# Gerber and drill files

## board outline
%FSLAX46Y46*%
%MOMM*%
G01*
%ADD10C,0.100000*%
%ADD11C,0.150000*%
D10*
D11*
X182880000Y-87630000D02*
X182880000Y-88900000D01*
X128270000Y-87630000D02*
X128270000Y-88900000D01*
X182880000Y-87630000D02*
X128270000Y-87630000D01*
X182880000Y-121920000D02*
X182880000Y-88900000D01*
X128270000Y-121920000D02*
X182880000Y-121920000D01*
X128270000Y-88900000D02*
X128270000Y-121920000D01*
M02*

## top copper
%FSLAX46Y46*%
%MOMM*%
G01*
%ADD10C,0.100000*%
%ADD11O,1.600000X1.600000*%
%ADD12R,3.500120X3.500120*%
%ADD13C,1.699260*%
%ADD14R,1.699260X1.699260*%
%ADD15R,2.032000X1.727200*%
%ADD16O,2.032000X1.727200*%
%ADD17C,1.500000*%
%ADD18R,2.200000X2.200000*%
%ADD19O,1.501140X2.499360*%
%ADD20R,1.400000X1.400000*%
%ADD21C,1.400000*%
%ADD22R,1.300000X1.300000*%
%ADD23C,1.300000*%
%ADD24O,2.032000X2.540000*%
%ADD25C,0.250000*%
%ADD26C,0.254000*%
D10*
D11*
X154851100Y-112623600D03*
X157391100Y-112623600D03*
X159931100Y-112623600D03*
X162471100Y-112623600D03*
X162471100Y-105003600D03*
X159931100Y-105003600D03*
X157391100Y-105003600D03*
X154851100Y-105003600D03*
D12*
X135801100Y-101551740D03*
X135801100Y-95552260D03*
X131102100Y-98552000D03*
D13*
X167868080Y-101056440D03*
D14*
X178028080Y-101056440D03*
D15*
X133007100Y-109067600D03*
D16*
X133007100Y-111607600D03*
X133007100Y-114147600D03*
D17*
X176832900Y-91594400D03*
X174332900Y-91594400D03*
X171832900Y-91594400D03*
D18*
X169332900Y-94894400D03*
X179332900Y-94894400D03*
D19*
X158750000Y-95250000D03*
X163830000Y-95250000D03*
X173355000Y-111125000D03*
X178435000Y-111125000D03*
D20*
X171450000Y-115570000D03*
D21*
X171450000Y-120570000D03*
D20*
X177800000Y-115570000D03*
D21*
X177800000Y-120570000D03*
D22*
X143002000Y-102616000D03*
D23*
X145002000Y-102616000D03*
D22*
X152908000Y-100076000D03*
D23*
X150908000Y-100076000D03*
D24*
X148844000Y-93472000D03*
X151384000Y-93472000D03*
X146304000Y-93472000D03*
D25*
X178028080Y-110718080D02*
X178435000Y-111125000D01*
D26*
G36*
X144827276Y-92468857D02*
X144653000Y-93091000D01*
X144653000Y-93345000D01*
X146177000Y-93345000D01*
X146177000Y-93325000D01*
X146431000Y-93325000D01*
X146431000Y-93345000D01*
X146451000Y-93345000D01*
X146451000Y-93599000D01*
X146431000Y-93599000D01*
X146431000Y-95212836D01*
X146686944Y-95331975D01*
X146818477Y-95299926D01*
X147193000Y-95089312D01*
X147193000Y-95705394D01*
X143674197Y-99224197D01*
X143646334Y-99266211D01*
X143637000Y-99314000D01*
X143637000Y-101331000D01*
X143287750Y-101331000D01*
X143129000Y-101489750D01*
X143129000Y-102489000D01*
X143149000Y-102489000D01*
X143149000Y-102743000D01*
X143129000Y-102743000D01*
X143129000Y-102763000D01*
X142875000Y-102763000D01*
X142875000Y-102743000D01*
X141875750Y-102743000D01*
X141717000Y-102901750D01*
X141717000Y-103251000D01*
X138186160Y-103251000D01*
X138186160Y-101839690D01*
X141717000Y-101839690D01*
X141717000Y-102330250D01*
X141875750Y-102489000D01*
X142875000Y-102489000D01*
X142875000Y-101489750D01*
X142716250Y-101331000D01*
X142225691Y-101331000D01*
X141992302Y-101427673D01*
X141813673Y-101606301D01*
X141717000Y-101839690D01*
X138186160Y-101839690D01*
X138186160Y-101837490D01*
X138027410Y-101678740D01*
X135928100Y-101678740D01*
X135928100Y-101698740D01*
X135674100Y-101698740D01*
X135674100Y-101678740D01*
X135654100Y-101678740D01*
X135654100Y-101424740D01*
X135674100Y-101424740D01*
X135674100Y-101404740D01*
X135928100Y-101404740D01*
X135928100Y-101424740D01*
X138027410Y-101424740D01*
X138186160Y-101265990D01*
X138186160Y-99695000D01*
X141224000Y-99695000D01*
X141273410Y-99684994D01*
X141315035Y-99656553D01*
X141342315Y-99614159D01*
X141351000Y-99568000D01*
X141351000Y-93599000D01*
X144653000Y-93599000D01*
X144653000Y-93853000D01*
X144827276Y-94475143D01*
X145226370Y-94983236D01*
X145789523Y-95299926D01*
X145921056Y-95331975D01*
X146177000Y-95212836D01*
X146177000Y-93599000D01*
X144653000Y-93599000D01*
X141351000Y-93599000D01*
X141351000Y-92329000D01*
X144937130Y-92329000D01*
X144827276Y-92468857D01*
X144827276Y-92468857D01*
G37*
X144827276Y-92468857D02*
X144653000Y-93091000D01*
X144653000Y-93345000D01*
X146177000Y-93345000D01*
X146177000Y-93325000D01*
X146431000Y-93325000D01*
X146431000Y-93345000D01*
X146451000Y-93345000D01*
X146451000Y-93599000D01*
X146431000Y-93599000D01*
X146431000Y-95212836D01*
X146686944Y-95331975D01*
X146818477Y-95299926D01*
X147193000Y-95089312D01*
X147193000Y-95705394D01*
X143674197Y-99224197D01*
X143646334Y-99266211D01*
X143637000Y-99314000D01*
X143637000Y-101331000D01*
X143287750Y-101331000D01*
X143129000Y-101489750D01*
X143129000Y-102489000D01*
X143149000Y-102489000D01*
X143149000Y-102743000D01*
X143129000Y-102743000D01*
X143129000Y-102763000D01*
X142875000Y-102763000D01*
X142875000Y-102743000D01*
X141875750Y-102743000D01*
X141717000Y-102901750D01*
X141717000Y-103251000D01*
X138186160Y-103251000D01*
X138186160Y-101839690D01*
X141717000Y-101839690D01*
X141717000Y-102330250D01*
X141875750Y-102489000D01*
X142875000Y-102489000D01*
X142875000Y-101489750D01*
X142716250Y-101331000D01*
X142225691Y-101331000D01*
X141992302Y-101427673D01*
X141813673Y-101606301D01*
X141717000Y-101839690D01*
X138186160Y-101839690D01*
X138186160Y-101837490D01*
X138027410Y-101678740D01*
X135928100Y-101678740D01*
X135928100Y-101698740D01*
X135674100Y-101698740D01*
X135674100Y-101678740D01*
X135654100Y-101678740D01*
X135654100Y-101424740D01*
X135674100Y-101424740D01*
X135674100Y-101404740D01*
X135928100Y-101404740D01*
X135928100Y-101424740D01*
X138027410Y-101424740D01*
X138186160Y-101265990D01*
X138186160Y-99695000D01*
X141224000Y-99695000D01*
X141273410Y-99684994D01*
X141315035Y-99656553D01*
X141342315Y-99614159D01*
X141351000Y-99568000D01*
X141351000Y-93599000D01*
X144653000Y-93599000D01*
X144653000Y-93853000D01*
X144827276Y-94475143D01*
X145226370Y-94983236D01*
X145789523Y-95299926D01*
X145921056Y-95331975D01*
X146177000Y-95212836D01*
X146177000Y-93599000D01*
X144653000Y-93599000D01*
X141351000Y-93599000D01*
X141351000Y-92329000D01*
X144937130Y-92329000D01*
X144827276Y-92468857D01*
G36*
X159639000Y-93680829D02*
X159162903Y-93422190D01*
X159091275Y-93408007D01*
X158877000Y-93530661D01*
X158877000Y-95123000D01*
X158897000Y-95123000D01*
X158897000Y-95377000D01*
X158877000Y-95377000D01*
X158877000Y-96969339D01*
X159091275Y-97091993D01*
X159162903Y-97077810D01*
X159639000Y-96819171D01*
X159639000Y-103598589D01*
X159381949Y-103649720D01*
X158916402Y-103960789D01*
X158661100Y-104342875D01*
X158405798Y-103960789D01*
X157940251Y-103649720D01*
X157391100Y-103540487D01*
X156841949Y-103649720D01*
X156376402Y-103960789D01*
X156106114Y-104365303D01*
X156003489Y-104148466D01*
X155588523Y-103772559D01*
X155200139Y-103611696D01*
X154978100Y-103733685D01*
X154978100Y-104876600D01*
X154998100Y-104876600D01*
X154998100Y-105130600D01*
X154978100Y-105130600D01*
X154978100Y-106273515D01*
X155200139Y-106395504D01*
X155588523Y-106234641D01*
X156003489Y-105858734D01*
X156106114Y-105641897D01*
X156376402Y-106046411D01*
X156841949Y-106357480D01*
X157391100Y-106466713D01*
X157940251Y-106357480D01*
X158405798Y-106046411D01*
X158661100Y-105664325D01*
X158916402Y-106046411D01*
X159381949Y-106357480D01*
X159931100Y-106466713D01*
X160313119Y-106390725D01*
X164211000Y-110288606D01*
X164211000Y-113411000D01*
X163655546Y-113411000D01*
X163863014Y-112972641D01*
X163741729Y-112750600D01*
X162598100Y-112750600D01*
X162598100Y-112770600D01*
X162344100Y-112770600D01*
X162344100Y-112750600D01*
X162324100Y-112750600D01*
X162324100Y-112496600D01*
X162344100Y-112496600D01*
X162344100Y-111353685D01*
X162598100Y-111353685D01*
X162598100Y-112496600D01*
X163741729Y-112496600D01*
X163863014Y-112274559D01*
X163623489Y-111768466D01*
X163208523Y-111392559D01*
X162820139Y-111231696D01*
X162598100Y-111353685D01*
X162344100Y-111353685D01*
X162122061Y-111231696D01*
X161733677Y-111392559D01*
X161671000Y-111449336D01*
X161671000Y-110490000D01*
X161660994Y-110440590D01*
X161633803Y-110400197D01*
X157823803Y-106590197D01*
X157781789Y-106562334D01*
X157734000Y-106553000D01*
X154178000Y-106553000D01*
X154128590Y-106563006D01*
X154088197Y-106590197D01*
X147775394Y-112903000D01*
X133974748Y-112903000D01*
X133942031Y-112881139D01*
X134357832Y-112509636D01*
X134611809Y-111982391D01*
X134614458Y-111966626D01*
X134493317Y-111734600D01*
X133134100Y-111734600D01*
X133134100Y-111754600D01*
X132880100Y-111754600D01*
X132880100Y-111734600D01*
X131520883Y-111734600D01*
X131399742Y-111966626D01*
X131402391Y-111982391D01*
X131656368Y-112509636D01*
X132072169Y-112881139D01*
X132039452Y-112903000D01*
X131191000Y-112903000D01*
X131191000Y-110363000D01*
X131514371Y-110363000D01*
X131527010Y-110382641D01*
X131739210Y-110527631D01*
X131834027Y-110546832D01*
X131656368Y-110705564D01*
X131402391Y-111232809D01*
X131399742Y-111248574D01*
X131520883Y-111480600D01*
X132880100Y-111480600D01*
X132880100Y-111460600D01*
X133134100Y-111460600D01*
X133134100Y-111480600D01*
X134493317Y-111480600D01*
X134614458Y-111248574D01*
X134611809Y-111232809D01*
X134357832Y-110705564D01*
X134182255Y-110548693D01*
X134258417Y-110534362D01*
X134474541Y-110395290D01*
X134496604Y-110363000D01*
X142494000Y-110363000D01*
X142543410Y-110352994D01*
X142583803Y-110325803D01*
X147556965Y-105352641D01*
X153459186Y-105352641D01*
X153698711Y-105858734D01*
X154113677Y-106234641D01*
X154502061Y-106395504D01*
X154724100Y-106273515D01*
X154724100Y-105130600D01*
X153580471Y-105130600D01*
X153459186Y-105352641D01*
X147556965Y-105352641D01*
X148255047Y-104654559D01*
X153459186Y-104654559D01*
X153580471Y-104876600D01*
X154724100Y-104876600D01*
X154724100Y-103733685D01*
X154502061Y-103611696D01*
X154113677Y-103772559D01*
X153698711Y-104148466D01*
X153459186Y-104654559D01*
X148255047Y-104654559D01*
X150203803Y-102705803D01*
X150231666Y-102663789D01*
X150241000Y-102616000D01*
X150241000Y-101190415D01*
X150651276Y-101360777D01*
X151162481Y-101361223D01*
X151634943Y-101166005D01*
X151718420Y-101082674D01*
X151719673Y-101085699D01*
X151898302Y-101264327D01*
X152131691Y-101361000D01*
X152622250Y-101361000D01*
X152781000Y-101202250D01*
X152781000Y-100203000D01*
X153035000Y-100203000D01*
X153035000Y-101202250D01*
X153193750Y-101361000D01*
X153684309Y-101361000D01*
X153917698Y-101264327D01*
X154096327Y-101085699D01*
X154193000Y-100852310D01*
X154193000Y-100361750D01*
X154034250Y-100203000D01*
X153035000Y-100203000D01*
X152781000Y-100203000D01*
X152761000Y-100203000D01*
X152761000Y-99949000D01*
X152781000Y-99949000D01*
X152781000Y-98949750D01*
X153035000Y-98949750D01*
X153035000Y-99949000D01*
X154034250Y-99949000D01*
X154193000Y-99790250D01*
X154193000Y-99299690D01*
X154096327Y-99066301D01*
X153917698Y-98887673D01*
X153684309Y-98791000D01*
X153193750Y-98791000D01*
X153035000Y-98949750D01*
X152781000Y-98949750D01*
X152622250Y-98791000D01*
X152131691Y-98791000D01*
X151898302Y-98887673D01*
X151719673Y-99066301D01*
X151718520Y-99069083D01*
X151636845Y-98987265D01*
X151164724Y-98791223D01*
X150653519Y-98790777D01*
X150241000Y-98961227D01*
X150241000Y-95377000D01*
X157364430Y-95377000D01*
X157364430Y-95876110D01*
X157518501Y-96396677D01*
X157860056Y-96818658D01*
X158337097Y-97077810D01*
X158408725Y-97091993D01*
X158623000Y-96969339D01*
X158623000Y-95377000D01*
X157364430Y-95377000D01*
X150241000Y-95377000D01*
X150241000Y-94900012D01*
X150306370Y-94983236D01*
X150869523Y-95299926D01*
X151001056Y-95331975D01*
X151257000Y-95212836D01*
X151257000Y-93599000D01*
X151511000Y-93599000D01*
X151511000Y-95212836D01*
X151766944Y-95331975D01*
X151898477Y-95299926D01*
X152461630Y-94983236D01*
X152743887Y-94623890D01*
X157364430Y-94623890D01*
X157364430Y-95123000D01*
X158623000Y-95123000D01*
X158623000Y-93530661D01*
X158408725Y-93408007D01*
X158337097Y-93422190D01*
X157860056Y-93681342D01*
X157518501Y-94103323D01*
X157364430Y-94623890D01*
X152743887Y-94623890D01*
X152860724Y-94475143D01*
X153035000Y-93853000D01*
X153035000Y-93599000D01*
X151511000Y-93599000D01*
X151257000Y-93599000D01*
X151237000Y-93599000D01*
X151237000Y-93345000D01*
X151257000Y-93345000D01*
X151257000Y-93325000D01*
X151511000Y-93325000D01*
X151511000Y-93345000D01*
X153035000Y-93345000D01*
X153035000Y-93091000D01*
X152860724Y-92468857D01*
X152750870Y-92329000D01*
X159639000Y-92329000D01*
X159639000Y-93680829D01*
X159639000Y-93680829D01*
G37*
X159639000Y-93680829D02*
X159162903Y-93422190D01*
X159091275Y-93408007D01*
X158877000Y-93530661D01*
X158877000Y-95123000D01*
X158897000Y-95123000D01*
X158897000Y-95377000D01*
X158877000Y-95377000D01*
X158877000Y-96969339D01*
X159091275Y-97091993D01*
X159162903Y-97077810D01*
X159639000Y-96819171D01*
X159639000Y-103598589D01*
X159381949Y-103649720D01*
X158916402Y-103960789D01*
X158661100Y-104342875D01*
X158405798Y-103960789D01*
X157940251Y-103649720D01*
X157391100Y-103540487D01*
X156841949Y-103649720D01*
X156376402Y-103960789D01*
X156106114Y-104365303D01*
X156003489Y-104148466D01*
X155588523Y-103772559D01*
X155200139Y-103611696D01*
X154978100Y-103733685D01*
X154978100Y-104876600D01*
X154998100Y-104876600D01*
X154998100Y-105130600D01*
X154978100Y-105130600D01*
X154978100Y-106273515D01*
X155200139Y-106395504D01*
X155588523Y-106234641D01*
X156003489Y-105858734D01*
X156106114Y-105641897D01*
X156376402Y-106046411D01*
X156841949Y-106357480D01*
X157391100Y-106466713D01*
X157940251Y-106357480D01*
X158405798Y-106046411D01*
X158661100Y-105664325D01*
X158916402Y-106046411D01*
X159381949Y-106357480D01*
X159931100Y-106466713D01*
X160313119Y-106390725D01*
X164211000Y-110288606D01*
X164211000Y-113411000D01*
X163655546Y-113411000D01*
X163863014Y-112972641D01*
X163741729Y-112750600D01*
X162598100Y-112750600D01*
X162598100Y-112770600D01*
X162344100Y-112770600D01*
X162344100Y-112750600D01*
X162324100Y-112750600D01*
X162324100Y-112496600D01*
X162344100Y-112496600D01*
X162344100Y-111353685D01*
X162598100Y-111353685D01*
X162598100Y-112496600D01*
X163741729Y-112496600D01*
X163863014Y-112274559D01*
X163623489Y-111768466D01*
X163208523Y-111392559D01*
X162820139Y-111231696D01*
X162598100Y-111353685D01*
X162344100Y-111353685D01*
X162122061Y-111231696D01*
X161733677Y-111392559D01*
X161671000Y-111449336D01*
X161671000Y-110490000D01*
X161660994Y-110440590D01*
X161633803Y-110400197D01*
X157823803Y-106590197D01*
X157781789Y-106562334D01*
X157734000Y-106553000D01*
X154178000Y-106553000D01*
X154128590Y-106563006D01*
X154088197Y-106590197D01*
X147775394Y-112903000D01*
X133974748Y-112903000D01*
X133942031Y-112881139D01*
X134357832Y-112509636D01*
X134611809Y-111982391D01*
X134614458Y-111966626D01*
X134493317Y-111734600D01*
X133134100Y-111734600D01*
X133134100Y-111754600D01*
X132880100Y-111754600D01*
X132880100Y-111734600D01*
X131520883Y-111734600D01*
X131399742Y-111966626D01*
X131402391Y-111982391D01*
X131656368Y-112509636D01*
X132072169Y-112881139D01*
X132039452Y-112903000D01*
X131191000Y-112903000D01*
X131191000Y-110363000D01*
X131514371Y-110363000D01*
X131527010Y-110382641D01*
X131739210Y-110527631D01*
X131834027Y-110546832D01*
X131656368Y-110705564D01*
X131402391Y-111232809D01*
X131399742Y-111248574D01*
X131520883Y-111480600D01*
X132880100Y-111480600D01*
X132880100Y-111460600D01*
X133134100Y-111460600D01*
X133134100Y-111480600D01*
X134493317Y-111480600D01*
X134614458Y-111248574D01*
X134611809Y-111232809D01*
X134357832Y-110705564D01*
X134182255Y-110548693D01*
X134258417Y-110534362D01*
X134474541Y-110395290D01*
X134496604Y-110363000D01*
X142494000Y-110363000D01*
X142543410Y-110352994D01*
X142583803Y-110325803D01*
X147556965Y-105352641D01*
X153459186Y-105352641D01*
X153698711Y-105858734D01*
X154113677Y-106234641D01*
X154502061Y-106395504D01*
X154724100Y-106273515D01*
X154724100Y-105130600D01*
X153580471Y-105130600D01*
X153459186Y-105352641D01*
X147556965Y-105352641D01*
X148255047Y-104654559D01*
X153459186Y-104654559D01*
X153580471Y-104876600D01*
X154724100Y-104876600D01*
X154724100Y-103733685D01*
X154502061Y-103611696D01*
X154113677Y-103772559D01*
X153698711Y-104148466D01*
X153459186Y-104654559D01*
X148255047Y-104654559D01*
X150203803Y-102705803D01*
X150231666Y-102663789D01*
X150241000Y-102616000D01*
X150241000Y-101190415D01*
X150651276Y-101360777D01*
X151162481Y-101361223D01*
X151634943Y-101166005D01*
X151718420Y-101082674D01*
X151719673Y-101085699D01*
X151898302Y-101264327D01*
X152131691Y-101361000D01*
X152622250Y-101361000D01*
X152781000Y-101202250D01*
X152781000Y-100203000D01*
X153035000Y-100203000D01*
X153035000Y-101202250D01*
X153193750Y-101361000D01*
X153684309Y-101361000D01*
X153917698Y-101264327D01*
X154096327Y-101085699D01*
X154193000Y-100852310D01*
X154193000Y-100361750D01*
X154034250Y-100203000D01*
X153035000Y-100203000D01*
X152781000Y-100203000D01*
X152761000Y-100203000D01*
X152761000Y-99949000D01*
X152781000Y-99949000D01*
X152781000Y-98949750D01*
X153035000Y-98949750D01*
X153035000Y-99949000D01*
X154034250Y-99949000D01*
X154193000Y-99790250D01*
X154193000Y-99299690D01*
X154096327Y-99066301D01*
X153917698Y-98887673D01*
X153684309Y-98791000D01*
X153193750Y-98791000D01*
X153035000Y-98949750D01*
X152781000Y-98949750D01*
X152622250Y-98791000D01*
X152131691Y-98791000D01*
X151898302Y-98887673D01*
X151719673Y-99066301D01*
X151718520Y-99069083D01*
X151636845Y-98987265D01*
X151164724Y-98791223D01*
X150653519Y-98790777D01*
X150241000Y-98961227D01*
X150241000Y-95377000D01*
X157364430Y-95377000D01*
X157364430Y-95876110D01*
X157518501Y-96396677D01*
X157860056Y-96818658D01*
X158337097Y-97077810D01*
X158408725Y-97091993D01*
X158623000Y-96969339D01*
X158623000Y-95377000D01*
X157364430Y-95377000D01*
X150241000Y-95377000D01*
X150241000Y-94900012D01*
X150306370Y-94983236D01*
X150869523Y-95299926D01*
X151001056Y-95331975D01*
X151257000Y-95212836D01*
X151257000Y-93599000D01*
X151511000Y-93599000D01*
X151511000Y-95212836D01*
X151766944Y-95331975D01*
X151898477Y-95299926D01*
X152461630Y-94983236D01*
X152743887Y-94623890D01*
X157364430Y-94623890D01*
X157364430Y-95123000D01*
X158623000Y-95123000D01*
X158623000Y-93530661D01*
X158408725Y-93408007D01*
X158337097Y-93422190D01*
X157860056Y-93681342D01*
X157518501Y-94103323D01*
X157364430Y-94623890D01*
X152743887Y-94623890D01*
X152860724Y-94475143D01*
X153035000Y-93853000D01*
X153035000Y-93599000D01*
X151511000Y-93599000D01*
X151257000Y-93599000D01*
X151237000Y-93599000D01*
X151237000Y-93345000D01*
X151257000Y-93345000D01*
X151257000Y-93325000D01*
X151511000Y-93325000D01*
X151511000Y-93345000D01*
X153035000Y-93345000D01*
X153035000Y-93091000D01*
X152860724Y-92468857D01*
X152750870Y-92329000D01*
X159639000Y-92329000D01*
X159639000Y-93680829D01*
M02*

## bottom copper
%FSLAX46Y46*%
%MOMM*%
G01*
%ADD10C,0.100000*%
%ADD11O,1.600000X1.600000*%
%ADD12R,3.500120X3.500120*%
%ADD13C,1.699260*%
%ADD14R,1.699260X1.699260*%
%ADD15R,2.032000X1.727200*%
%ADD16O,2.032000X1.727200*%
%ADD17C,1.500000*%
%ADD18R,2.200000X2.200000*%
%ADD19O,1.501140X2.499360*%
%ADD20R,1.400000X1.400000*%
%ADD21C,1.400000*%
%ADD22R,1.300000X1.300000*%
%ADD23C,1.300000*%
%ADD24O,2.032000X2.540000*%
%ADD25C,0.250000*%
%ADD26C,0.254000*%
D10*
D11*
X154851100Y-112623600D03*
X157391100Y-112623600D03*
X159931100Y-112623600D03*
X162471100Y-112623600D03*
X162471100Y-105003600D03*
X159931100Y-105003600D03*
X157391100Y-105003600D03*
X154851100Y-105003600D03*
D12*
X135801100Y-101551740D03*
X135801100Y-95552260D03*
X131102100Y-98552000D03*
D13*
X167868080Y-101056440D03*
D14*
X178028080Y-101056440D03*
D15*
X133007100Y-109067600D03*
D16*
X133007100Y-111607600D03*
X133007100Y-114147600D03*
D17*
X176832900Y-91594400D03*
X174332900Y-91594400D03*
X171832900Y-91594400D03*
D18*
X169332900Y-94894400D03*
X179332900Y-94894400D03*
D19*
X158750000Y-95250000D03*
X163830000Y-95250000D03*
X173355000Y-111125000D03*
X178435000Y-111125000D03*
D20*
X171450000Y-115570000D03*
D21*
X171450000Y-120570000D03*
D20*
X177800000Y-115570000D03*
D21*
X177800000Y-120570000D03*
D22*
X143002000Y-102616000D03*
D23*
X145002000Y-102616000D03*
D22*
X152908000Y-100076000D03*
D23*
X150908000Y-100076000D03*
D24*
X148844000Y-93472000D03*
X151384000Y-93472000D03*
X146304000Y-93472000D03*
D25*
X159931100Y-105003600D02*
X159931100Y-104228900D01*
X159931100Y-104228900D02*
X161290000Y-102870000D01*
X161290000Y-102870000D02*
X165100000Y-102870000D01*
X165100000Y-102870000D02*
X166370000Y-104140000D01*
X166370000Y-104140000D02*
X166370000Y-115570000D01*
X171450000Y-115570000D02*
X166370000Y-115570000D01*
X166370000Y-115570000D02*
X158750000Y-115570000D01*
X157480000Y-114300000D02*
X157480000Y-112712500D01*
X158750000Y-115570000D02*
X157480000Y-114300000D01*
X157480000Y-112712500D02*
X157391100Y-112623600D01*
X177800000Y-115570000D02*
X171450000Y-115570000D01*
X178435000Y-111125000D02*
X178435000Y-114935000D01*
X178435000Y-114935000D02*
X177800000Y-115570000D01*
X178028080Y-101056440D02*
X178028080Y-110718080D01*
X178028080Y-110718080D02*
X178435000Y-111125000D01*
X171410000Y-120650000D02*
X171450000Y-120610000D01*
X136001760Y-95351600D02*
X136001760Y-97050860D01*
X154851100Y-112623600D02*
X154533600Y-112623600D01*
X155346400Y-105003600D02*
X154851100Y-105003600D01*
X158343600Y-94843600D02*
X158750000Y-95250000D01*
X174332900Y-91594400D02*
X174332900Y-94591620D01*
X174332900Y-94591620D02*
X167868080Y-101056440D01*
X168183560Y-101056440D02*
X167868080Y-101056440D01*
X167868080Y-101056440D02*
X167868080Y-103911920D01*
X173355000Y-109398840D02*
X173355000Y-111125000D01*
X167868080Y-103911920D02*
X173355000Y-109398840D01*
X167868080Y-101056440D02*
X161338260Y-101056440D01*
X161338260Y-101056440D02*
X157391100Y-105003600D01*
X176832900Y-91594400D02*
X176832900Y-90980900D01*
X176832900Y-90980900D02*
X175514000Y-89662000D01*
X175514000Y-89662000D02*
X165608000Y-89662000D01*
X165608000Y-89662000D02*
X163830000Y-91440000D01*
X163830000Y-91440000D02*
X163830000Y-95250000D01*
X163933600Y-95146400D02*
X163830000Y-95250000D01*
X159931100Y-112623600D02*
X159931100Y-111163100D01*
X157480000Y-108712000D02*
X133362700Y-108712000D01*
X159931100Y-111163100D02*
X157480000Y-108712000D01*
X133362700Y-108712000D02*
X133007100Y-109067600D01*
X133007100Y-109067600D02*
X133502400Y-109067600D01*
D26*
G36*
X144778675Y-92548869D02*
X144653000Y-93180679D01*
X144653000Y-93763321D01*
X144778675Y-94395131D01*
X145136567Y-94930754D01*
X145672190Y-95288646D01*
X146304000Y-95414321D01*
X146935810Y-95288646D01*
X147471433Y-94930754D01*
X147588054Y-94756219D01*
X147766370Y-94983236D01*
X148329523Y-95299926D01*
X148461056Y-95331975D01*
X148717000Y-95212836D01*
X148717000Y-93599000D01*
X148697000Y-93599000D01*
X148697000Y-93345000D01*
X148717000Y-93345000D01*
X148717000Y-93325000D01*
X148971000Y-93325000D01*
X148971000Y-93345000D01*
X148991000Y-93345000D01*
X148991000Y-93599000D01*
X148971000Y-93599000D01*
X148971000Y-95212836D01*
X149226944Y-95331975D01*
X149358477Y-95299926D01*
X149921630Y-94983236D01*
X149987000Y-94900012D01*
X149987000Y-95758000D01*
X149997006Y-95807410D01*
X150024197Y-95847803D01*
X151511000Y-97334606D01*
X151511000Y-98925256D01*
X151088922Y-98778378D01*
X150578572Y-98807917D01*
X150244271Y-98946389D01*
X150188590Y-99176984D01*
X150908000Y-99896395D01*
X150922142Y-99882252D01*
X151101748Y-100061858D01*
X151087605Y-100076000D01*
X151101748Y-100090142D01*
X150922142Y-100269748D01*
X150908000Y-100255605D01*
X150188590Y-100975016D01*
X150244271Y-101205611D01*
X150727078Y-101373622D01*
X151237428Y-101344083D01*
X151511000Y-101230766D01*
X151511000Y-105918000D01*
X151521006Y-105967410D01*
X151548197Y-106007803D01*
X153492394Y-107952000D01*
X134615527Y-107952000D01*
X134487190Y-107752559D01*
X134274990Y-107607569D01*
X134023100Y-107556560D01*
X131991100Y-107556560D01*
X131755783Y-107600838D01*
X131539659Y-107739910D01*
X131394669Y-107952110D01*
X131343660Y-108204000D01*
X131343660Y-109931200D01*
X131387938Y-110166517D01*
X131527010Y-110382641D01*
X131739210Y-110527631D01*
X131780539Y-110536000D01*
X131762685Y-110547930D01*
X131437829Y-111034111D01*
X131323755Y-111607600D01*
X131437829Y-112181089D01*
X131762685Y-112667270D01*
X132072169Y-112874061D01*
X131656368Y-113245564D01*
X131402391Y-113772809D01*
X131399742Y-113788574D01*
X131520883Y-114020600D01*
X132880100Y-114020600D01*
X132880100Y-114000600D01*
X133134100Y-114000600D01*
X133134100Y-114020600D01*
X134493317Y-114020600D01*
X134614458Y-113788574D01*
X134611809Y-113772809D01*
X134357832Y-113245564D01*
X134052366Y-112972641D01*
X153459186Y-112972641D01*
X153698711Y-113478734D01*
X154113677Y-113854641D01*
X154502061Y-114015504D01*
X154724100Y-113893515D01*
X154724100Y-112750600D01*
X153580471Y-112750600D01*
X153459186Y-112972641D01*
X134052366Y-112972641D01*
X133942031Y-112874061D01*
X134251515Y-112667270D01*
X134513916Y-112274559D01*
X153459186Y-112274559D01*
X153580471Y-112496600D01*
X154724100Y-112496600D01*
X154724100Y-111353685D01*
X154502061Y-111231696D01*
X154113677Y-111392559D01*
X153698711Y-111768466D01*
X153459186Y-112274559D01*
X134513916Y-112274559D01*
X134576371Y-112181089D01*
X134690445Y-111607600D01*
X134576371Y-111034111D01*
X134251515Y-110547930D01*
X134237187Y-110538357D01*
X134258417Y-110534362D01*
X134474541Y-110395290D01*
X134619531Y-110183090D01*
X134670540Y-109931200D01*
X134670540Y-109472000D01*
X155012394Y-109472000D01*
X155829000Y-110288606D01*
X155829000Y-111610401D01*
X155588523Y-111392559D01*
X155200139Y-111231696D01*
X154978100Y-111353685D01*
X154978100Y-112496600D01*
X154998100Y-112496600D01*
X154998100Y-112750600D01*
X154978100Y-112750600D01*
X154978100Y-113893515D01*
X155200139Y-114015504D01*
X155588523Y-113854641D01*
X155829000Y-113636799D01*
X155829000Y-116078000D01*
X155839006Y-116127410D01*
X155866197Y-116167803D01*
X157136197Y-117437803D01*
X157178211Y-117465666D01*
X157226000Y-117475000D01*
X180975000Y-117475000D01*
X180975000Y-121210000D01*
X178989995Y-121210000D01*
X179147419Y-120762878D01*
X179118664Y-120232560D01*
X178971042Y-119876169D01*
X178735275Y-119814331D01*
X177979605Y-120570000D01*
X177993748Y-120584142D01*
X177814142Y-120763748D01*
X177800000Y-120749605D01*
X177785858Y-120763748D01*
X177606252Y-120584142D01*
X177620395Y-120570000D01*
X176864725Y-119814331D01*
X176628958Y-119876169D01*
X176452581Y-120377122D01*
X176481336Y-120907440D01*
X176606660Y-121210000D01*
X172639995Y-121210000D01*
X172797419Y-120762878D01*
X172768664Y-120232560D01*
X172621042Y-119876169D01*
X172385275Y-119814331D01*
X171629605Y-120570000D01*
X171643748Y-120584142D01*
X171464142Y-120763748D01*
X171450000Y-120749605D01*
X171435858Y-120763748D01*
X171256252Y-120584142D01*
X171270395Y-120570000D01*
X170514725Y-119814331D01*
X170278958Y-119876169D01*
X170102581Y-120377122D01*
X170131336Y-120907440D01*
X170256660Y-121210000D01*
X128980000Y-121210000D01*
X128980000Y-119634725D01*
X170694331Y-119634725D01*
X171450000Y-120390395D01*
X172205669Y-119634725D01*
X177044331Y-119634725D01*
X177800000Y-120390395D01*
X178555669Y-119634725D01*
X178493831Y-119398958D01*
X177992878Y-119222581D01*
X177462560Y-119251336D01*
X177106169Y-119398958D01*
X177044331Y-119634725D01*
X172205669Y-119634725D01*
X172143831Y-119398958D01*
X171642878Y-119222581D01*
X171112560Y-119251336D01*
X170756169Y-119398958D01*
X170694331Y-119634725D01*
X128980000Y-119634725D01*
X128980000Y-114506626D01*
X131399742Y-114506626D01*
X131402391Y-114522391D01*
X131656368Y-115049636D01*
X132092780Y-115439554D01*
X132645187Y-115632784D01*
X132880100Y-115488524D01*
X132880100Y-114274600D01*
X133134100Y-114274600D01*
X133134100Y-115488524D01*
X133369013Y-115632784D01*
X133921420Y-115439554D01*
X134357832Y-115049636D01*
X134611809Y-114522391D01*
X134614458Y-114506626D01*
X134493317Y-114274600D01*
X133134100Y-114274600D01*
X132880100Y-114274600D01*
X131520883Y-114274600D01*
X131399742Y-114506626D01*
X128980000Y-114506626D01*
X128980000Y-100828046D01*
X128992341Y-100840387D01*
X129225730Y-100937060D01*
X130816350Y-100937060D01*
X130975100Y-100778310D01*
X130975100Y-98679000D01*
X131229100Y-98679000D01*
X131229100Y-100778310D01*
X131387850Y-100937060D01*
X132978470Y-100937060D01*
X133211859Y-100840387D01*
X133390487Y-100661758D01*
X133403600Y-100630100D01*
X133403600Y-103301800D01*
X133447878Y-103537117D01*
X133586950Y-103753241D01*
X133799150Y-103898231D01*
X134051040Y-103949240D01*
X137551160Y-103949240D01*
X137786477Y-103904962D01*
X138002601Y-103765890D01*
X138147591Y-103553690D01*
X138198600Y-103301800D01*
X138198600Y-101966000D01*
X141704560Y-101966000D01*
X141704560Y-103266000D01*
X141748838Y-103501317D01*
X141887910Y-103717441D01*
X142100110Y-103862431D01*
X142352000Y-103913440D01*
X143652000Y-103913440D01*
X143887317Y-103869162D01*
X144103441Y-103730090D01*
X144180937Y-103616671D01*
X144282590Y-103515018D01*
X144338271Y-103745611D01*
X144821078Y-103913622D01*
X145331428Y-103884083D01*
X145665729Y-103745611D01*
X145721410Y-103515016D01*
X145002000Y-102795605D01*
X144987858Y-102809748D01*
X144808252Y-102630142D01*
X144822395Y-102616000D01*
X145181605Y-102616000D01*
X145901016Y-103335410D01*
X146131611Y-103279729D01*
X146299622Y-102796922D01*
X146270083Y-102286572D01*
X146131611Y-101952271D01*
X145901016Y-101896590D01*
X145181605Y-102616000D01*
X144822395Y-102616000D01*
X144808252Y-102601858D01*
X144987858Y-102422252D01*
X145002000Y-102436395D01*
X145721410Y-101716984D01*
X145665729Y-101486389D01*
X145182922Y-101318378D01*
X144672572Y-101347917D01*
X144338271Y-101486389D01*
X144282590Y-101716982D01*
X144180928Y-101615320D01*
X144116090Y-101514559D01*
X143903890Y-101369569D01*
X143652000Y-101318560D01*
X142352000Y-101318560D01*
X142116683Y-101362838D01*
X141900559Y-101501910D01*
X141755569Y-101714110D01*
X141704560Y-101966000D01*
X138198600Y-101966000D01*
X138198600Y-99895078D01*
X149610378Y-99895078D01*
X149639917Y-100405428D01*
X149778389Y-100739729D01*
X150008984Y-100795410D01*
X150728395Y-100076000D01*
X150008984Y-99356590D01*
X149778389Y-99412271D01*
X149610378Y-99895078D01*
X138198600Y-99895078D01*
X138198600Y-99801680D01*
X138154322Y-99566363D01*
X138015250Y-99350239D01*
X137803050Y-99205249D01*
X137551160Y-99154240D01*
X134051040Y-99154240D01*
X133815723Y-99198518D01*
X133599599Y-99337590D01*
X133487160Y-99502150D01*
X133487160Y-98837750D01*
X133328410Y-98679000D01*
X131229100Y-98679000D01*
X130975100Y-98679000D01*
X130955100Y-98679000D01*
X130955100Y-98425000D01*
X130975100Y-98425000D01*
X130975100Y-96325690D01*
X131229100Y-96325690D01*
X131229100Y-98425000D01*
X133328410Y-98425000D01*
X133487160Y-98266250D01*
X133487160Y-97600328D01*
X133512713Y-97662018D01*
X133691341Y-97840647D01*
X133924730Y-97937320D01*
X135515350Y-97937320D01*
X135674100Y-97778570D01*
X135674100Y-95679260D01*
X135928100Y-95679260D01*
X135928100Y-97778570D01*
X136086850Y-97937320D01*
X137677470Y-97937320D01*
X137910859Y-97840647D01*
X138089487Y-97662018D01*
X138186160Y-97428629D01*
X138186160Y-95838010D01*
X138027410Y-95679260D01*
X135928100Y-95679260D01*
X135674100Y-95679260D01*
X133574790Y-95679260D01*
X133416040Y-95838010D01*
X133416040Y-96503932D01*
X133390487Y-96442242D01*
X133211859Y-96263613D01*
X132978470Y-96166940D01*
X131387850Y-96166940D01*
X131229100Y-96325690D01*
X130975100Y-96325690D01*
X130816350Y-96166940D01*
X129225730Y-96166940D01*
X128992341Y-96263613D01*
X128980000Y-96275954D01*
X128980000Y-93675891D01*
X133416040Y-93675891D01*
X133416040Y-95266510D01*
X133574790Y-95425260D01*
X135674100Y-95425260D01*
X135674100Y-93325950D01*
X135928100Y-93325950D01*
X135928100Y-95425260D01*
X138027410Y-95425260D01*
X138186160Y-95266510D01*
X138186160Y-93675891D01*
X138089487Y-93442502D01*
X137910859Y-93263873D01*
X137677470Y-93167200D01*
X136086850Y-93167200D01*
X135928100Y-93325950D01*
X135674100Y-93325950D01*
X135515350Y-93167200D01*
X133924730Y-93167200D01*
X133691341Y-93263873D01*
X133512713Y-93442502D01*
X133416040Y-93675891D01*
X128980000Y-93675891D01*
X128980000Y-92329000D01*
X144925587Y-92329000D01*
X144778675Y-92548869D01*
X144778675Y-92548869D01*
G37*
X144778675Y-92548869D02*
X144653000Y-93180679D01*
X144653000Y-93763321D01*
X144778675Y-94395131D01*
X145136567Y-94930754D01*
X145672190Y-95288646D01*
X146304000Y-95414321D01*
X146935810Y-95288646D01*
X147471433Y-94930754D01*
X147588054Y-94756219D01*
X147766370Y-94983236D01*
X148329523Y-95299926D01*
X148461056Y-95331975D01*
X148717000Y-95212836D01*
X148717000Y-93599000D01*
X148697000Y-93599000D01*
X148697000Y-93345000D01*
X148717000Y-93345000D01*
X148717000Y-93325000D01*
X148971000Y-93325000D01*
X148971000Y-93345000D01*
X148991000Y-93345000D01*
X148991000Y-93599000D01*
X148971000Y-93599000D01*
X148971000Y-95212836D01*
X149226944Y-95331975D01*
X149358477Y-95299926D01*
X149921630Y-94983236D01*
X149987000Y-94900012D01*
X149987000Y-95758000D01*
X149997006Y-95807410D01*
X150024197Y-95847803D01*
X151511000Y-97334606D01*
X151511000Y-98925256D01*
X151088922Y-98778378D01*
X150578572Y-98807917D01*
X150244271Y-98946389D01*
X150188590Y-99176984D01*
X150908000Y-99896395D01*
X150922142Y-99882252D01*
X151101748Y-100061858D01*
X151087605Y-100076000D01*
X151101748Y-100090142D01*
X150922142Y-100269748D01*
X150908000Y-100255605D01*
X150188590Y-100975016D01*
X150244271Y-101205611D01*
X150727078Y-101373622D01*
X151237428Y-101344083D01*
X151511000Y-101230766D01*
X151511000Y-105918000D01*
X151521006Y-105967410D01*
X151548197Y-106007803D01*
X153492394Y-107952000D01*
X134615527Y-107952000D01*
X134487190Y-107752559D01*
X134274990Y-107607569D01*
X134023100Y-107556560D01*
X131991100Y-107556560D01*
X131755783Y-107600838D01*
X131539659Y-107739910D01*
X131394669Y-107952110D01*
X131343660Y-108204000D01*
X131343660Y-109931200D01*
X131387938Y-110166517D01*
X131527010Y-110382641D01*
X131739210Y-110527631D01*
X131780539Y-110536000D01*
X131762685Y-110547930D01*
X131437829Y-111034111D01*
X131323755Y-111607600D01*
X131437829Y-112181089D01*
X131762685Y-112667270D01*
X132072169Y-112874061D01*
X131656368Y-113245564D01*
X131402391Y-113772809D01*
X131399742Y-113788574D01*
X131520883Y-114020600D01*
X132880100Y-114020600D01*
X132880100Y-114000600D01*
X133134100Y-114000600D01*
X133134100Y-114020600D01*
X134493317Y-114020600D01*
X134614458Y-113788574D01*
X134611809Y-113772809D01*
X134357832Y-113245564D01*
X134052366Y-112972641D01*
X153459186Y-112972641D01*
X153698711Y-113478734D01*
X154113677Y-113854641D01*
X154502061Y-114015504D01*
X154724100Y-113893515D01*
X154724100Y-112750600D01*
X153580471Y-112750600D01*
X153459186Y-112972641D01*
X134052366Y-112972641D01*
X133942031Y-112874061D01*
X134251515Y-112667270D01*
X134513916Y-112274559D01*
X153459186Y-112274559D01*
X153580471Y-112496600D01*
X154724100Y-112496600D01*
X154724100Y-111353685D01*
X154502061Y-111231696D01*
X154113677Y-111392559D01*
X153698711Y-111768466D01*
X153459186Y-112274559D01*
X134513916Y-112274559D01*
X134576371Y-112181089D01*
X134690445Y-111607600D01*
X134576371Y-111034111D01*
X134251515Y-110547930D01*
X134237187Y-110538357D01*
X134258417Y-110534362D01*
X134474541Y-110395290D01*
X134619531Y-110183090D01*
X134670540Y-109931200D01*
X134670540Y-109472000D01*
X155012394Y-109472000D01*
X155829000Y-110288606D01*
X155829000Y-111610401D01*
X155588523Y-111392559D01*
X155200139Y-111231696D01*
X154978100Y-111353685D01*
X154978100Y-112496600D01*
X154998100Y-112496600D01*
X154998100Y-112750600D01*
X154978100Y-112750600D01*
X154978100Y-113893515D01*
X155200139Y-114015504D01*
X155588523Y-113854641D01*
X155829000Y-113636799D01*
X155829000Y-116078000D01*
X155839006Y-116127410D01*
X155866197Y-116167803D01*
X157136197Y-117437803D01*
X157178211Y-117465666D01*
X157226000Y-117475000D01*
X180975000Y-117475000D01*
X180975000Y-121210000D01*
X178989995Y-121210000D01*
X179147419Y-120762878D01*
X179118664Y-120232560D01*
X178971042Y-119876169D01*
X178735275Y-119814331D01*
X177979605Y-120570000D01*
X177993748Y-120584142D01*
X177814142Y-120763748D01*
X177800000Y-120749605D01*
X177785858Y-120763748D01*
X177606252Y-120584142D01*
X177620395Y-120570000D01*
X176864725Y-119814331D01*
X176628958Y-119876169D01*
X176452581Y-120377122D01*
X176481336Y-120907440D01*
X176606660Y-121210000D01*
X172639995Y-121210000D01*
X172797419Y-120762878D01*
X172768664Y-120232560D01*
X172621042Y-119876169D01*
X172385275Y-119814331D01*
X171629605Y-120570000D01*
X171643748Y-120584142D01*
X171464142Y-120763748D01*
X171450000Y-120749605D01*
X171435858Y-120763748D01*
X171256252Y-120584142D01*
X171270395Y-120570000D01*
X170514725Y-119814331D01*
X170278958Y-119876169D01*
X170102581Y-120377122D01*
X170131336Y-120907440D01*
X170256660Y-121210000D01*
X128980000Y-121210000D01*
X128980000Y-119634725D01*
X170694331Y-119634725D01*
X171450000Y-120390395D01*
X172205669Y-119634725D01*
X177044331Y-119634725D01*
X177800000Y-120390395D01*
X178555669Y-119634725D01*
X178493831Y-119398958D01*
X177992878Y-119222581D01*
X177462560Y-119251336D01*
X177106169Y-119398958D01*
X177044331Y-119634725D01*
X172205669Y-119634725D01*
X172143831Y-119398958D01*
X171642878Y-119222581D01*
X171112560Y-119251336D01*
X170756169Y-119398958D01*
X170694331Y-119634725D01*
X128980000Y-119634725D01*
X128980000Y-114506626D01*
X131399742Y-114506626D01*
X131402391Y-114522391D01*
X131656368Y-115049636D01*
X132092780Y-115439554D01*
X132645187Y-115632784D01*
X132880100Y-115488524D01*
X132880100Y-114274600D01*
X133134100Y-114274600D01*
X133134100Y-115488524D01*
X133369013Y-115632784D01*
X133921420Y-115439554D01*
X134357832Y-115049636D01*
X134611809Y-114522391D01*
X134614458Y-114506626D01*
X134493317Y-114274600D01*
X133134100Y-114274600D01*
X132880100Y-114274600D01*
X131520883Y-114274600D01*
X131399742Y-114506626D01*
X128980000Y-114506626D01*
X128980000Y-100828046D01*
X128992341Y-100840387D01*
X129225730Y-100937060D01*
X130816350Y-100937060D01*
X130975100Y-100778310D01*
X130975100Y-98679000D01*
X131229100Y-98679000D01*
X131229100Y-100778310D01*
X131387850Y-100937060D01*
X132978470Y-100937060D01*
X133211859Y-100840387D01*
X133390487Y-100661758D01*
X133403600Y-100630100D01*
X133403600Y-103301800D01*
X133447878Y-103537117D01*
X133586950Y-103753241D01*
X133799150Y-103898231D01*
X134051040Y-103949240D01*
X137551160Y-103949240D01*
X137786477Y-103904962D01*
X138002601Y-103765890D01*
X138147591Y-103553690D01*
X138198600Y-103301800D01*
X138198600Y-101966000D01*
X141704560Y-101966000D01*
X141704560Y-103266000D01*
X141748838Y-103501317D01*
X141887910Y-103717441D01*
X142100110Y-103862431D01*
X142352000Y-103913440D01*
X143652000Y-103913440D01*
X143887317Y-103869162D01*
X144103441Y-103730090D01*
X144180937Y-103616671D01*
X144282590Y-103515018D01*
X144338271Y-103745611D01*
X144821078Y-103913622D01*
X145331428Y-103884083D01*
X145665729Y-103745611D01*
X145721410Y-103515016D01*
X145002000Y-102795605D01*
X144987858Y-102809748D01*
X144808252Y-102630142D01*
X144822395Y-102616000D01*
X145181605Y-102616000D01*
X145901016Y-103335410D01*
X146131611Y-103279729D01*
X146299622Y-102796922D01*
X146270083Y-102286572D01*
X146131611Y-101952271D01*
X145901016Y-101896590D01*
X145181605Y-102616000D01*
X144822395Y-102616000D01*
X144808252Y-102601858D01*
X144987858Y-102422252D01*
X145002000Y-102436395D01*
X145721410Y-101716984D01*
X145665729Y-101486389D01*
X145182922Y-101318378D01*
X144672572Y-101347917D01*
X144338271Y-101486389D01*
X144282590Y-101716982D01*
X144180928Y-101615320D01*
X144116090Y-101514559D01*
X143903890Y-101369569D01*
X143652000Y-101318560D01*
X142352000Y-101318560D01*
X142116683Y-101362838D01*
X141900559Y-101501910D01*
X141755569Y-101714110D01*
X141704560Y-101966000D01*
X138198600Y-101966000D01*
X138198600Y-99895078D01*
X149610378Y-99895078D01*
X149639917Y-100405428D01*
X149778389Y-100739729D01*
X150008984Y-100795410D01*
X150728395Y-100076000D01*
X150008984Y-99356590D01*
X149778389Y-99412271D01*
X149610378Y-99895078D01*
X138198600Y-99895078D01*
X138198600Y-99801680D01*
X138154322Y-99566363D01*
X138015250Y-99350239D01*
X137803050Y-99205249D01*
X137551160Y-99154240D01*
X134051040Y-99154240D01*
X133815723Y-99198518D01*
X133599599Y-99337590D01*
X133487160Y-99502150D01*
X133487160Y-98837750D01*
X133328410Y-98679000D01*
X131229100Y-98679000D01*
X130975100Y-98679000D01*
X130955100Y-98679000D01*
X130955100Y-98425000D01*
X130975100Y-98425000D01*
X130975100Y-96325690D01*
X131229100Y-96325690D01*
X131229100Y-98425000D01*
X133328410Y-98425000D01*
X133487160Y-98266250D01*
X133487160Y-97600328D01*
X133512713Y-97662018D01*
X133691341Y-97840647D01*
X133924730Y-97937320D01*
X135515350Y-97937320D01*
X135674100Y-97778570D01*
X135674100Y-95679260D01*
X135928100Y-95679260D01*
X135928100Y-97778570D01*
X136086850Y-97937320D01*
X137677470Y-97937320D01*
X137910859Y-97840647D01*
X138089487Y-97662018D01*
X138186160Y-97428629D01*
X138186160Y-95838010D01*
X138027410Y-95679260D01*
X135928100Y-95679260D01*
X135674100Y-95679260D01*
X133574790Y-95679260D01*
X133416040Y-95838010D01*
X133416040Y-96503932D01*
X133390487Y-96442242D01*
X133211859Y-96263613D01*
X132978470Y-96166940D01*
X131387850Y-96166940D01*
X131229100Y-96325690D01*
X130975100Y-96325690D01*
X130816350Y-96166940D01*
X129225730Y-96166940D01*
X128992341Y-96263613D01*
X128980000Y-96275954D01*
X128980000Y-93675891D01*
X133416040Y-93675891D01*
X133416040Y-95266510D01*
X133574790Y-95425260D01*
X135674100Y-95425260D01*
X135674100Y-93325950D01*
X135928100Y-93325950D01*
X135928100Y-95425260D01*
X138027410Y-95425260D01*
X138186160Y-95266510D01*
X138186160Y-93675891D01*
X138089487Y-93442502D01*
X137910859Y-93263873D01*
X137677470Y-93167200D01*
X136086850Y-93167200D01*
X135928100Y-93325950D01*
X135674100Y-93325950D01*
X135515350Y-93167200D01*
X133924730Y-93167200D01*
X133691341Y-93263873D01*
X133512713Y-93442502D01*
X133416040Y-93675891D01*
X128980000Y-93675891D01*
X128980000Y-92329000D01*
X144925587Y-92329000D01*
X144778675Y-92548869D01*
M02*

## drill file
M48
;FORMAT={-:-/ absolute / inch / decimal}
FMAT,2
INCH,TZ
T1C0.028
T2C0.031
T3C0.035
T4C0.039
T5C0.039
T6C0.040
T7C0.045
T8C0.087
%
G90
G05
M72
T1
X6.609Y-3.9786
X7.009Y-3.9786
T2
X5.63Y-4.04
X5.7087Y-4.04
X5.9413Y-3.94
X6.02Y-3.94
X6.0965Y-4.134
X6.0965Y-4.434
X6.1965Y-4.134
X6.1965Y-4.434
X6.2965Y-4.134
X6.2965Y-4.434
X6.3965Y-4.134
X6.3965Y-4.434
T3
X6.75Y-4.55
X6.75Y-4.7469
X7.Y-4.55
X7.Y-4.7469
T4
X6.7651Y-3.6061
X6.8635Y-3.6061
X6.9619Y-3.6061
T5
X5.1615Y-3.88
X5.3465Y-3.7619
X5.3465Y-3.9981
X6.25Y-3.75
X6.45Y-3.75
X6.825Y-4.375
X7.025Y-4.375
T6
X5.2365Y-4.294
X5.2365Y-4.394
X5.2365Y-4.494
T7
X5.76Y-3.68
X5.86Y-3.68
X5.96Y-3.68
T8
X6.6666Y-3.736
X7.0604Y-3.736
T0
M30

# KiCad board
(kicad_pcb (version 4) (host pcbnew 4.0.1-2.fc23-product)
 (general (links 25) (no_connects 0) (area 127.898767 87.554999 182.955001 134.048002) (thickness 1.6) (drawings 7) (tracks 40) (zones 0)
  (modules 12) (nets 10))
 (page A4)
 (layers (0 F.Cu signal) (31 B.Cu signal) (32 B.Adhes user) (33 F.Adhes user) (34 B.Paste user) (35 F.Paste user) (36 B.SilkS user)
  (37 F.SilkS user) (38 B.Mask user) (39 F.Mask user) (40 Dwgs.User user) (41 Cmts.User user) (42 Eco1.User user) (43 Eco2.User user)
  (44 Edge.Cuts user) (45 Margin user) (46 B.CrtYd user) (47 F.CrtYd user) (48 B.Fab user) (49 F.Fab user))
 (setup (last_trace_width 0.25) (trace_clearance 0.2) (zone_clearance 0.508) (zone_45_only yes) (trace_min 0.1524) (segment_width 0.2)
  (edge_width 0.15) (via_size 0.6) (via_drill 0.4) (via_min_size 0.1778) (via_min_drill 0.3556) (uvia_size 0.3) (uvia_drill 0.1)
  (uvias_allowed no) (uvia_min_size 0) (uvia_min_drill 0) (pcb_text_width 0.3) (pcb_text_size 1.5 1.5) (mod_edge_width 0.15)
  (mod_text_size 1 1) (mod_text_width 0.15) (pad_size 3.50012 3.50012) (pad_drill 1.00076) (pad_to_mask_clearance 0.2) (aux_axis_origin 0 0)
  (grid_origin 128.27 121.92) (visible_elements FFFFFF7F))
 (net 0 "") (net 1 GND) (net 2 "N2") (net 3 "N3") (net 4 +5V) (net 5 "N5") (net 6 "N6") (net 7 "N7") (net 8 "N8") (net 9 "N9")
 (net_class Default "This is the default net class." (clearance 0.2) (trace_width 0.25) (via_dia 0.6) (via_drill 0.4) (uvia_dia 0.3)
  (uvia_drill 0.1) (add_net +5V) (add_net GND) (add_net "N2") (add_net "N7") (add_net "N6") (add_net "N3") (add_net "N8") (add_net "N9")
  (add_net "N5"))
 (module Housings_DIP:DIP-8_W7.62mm (layer F.Cu) (at 154.8511 112.6236 90)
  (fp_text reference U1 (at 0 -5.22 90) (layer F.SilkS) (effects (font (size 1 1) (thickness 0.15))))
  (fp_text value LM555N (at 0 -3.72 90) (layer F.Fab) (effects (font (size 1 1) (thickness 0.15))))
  (pad 1 thru_hole oval (at 0 0 90) (size 1.6 1.6) (drill 0.8) (layers *.Cu *.Mask F.SilkS) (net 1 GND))
  (pad 2 thru_hole oval (at 0 2.54 90) (size 1.6 1.6) (drill 0.8) (layers *.Cu *.Mask F.SilkS) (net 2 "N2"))
  (pad 3 thru_hole oval (at 0 5.08 90) (size 1.6 1.6) (drill 0.8) (layers *.Cu *.Mask F.SilkS) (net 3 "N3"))
  (pad 4 thru_hole oval (at 0 7.62 90) (size 1.6 1.6) (drill 0.8) (layers *.Cu *.Mask F.SilkS) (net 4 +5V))
  (pad 5 thru_hole oval (at 7.62 7.62 90) (size 1.6 1.6) (drill 0.8) (layers *.Cu *.Mask F.SilkS) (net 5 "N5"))
  (pad 6 thru_hole oval (at 7.62 5.08 90) (size 1.6 1.6) (drill 0.8) (layers *.Cu *.Mask F.SilkS) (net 2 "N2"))
  (pad 7 thru_hole oval (at 7.62 2.54 90) (size 1.6 1.6) (drill 0.8) (layers *.Cu *.Mask F.SilkS) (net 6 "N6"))
  (pad 8 thru_hole oval (at 7.62 0 90) (size 1.6 1.6) (drill 0.8) (layers *.Cu *.Mask F.SilkS) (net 4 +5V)))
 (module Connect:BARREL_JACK (layer F.Cu) (at 135.8011 95.3516 270)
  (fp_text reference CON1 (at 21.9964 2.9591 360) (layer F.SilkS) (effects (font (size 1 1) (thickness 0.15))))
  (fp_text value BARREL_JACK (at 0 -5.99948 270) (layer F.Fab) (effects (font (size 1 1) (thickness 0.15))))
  (pad 1 thru_hole rect (at 6.20014 0 270) (size 3.50012 3.50012) (drill 1.00076) (layers *.Cu *.Mask F.SilkS) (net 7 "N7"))
  (pad 2 thru_hole rect (at 0.20066 0 270) (size 3.50012 3.50012) (drill 1.00076) (layers *.Cu *.Mask F.SilkS) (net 1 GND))
  (pad 3 thru_hole rect (at 3.2004 4.699 270) (size 3.50012 3.50012) (drill 1.00076) (layers *.Cu *.Mask F.SilkS) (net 1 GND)))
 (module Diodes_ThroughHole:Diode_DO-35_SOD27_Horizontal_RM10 (layer F.Cu) (at 178.0286 101.0539 180)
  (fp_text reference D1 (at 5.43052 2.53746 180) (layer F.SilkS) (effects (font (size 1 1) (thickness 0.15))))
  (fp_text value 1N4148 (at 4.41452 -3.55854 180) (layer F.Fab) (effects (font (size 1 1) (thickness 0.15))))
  (pad 2 thru_hole circle (at 10.16052 -0.00254) (size 1.69926 1.69926) (drill 0.70104) (layers *.Cu *.Mask F.SilkS) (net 6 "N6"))
  (pad 1 thru_hole rect (at 0.00052 -0.00254) (size 1.69926 1.69926) (drill 0.70104) (layers *.Cu *.Mask F.SilkS) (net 2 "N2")))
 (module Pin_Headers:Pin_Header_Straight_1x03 (layer F.Cu) (at 133.0071 109.0676)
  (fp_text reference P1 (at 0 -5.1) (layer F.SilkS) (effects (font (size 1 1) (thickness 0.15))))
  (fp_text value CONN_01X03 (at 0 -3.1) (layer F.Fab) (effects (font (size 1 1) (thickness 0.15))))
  (pad 1 thru_hole rect (at 0 0) (size 2.032 1.7272) (drill 1.016) (layers *.Cu *.Mask F.SilkS) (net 3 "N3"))
  (pad 2 thru_hole oval (at 0 2.54) (size 2.032 1.7272) (drill 1.016) (layers *.Cu *.Mask F.SilkS) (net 4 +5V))
  (pad 3 thru_hole oval (at 0 5.08) (size 2.032 1.7272) (drill 1.016) (layers *.Cu *.Mask F.SilkS) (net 1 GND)))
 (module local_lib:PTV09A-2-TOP (layer F.Cu) (at 174.3329 94.8944 180)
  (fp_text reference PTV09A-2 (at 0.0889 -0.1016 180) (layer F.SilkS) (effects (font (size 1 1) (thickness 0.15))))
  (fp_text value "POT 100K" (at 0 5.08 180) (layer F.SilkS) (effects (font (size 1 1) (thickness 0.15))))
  (pad 1 thru_hole circle (at -2.5 3.3) (size 1.5 1.5) (drill 1) (layers *.Cu *.Mask F.SilkS) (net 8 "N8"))
  (pad 2 thru_hole circle (at 0 3.3) (size 1.5 1.5) (drill 1) (layers *.Cu *.Mask F.SilkS) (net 6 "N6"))
  (pad 3 thru_hole circle (at 2.5 3.3) (size 1.5 1.5) (drill 1) (layers *.Cu *.Mask F.SilkS) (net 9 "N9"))
  (pad "" np_thru_hole rect (at 5 0 180) (size 2.2 2.2) (drill 2.2) (layers *.Cu *.Mask F.SilkS))
  (pad "" np_thru_hole rect (at -5 0 180) (size 2.2 2.2) (drill 2.2) (layers *.Cu *.Mask F.SilkS)))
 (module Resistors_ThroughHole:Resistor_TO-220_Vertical (layer F.Cu) (at 161.29 95.25)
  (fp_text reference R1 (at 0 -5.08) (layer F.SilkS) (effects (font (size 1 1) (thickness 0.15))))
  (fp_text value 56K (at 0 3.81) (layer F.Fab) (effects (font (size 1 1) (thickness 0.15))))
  (pad 1 thru_hole oval (at -2.54 0 90) (size 2.49936 1.50114) (drill 1.00076) (layers *.Cu *.Mask F.SilkS) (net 4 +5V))
  (pad 2 thru_hole oval (at 2.54 0 90) (size 2.49936 1.50114) (drill 1.00076) (layers *.Cu *.Mask F.SilkS) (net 8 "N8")))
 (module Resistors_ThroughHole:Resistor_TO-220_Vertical (layer F.Cu) (at 175.895 111.125)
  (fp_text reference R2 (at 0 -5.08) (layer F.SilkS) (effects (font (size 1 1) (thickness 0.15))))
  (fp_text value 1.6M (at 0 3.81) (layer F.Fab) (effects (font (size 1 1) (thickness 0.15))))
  (pad 1 thru_hole oval (at -2.54 0 90) (size 2.49936 1.50114) (drill 1.00076) (layers *.Cu *.Mask F.SilkS) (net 6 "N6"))
  (pad 2 thru_hole oval (at 2.54 0 90) (size 2.49936 1.50114) (drill 1.00076) (layers *.Cu *.Mask F.SilkS) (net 2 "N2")))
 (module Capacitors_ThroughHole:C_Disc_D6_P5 (layer F.Cu) (at 171.45 115.57 270)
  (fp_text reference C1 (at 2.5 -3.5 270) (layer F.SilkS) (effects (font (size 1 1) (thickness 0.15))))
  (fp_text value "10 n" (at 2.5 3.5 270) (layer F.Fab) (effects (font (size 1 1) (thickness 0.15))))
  (pad 1 thru_hole rect (at 0 0 270) (size 1.4 1.4) (drill 0.9) (layers *.Cu *.Mask F.SilkS) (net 2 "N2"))
  (pad 2 thru_hole circle (at 5 0 270) (size 1.4 1.4) (drill 0.9) (layers *.Cu *.Mask F.SilkS) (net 1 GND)))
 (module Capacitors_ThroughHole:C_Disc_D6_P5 (layer F.Cu) (at 177.8 115.57 270)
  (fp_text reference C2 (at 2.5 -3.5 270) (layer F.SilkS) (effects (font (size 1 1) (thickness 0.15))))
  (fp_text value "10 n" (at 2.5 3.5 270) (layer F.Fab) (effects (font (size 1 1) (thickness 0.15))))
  (pad 1 thru_hole rect (at 0 0 270) (size 1.4 1.4) (drill 0.9) (layers *.Cu *.Mask F.SilkS) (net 2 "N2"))
  (pad 2 thru_hole circle (at 5 0 270) (size 1.4 1.4) (drill 0.9) (layers *.Cu *.Mask F.SilkS) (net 1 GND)))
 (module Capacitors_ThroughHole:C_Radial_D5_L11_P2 (layer F.Cu) (at 143.002 102.616)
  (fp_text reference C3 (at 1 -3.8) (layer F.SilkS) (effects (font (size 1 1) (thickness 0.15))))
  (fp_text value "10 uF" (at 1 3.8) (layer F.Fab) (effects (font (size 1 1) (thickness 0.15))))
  (pad 1 thru_hole rect (at 0 0) (size 1.3 1.3) (drill 0.8) (layers *.Cu *.Mask F.SilkS) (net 7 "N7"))
  (pad 2 thru_hole circle (at 2 0) (size 1.3 1.3) (drill 0.8) (layers *.Cu *.Mask F.SilkS) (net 1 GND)))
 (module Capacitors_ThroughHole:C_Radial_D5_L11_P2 (layer F.Cu) (at 152.908 100.076 180)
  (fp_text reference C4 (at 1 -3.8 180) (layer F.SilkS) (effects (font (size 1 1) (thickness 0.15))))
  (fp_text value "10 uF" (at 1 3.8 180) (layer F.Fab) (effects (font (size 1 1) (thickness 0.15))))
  (pad 1 thru_hole rect (at 0 0 180) (size 1.3 1.3) (drill 0.8) (layers *.Cu *.Mask F.SilkS) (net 4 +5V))
  (pad 2 thru_hole circle (at 2 0 180) (size 1.3 1.3) (drill 0.8) (layers *.Cu *.Mask F.SilkS) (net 1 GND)))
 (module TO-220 (layer F.Cu) (at 148.844 93.472)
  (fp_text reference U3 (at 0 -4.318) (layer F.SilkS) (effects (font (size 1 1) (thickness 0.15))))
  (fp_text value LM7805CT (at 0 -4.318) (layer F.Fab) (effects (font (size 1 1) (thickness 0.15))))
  (pad 2 thru_hole oval (at 0 0) (size 2.032 2.54) (drill 1.143) (layers *.Cu *.Mask F.SilkS) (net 1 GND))
  (pad 3 thru_hole oval (at 2.54 0) (size 2.032 2.54) (drill 1.143) (layers *.Cu *.Mask F.SilkS) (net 4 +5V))
  (pad 1 thru_hole oval (at -2.54 0) (size 2.032 2.54) (drill 1.143) (layers *.Cu *.Mask F.SilkS) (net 7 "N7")))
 (gr_line (start 182.88 87.63) (end 182.88 88.9) (angle 90) (layer Edge.Cuts) (width 0.15))
 (gr_line (start 128.27 87.63) (end 128.27 88.9) (angle 90) (layer Edge.Cuts) (width 0.15))
 (gr_line (start 182.88 87.63) (end 128.27 87.63) (angle 90) (layer Edge.Cuts) (width 0.15))
 (gr_line (start 182.88 121.92) (end 182.88 88.9) (angle 90) (layer Edge.Cuts) (width 0.15))
 (gr_line (start 128.27 121.92) (end 182.88 121.92) (angle 90) (layer Edge.Cuts) (width 0.15))
 (gr_line (start 128.27 88.9) (end 128.27 121.92) (angle 90) (layer Edge.Cuts) (width 0.15))
 (segment (start 159.9311 105.0036) (end 159.9311 104.2289) (width 0.25) (layer B.Cu) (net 2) (status 30))
 (segment (start 159.9311 104.2289) (end 161.29 102.87) (width 0.25) (layer B.Cu) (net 2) (status 10))
 (segment (start 161.29 102.87) (end 165.1 102.87) (width 0.25) (layer B.Cu) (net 2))
 (segment (start 165.1 102.87) (end 166.37 104.14) (width 0.25) (layer B.Cu) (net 2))
 (segment (start 166.37 104.14) (end 166.37 115.57) (width 0.25) (layer B.Cu) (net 2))
 (segment (start 171.45 115.57) (end 166.37 115.57) (width 0.25) (layer B.Cu) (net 2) (status 10))
 (segment (start 166.37 115.57) (end 158.75 115.57) (width 0.25) (layer B.Cu) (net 2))
 (segment (start 157.48 114.3) (end 157.48 112.7125) (width 0.25) (layer B.Cu) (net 2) (status 20))
 (segment (start 158.75 115.57) (end 157.48 114.3) (width 0.25) (layer B.Cu) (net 2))
 (segment (start 157.48 112.7125) (end 157.3911 112.6236) (width 0.25) (layer B.Cu) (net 2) (status 30))
 (segment (start 177.8 115.57) (end 171.45 115.57) (width 0.25) (layer B.Cu) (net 2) (status 30))
 (segment (start 178.435 111.125) (end 178.435 114.935) (width 0.25) (layer B.Cu) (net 2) (status 30))
 (segment (start 178.435 114.935) (end 177.8 115.57) (width 0.25) (layer B.Cu) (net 2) (status 30))
 (segment (start 178.02808 101.05644) (end 178.02808 110.71808) (width 0.25) (layer B.Cu) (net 2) (status 30))
 (segment (start 178.02808 110.71808) (end 178.435 111.125) (width 0.25) (layer B.Cu) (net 2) (status 30))
 (segment (start 178.02808 110.71808) (end 178.435 111.125) (width 0.25) (layer F.Cu) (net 2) (status 30))
 (segment (start 171.41 120.65) (end 171.45 120.61) (width 0.25) (layer B.Cu) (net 1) (status 30))
 (segment (start 136.00176 95.3516) (end 136.00176 97.05086) (width 0.25) (layer B.Cu) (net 1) (status 30))
 (segment (start 154.8511 112.6236) (end 154.5336 112.6236) (width 0.25) (layer B.Cu) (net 1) (status 30))
 (segment (start 155.3464 105.0036) (end 154.8511 105.0036) (width 0.25) (layer B.Cu) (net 4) (status 30))
 (segment (start 158.3436 94.8436) (end 158.75 95.25) (width 0.25) (layer B.Cu) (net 4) (status 30))
 (segment (start 174.3329 91.5944) (end 174.3329 94.59162) (width 0.25) (layer B.Cu) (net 6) (status 10))
 (segment (start 174.3329 94.59162) (end 167.86808 101.05644) (width 0.25) (layer B.Cu) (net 6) (status 20))
 (segment (start 168.18356 101.05644) (end 167.86808 101.05644) (width 0.25) (layer B.Cu) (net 6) (status 30))
 (segment (start 167.86808 101.05644) (end 167.86808 103.91192) (width 0.25) (layer B.Cu) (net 6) (status 10))
 (segment (start 173.355 109.39884) (end 173.355 111.125) (width 0.25) (layer B.Cu) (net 6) (status 20))
 (segment (start 167.86808 103.91192) (end 173.355 109.39884) (width 0.25) (layer B.Cu) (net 6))
 (segment (start 167.86808 101.05644) (end 161.33826 101.05644) (width 0.25) (layer B.Cu) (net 6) (status 10))
 (segment (start 161.33826 101.05644) (end 157.3911 105.0036) (width 0.25) (layer B.Cu) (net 6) (status 20))
 (segment (start 176.8329 91.5944) (end 176.8329 90.9809) (width 0.25) (layer B.Cu) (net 8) (status 30))
 (segment (start 176.8329 90.9809) (end 175.514 89.662) (width 0.25) (layer B.Cu) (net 8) (status 10))
 (segment (start 175.514 89.662) (end 165.608 89.662) (width 0.25) (layer B.Cu) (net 8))
 (segment (start 165.608 89.662) (end 163.83 91.44) (width 0.25) (layer B.Cu) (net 8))
 (segment (start 163.83 91.44) (end 163.83 95.25) (width 0.25) (layer B.Cu) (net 8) (status 20))
 (segment (start 163.9336 95.1464) (end 163.83 95.25) (width 0.25) (layer B.Cu) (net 8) (status 30))
 (segment (start 159.9311 112.6236) (end 159.9311 111.1631) (width 0.25) (layer B.Cu) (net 3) (status 10))
 (segment (start 157.48 108.712) (end 133.3627 108.712) (width 0.25) (layer B.Cu) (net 3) (status 20))
 (segment (start 159.9311 111.1631) (end 157.48 108.712) (width 0.25) (layer B.Cu) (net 3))
 (segment (start 133.3627 108.712) (end 133.0071 109.0676) (width 0.25) (layer B.Cu) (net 3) (status 30))
 (segment (start 133.0071 109.0676) (end 133.5024 109.0676) (width 0.25) (layer B.Cu) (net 3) (status 30))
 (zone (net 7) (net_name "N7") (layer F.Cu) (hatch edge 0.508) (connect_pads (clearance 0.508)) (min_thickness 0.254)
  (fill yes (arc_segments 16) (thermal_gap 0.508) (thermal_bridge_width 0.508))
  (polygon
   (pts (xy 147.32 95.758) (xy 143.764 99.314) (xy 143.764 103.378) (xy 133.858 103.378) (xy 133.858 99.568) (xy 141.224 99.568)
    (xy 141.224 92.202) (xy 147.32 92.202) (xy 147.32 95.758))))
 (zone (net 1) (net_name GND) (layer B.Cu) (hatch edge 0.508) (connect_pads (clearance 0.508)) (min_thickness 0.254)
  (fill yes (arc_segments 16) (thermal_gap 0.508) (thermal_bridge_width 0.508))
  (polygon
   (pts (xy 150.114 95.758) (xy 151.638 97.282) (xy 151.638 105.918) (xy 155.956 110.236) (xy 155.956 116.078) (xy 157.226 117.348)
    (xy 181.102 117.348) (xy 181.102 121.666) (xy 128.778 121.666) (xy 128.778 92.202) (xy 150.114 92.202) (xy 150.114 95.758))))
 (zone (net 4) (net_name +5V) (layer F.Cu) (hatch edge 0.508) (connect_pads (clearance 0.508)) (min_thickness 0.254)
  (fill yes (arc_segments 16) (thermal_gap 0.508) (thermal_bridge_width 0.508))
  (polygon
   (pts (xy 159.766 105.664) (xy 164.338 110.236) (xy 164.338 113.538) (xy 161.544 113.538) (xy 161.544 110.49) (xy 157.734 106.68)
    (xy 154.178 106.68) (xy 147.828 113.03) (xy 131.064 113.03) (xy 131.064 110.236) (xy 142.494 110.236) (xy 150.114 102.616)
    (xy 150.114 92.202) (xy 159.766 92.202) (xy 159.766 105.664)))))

